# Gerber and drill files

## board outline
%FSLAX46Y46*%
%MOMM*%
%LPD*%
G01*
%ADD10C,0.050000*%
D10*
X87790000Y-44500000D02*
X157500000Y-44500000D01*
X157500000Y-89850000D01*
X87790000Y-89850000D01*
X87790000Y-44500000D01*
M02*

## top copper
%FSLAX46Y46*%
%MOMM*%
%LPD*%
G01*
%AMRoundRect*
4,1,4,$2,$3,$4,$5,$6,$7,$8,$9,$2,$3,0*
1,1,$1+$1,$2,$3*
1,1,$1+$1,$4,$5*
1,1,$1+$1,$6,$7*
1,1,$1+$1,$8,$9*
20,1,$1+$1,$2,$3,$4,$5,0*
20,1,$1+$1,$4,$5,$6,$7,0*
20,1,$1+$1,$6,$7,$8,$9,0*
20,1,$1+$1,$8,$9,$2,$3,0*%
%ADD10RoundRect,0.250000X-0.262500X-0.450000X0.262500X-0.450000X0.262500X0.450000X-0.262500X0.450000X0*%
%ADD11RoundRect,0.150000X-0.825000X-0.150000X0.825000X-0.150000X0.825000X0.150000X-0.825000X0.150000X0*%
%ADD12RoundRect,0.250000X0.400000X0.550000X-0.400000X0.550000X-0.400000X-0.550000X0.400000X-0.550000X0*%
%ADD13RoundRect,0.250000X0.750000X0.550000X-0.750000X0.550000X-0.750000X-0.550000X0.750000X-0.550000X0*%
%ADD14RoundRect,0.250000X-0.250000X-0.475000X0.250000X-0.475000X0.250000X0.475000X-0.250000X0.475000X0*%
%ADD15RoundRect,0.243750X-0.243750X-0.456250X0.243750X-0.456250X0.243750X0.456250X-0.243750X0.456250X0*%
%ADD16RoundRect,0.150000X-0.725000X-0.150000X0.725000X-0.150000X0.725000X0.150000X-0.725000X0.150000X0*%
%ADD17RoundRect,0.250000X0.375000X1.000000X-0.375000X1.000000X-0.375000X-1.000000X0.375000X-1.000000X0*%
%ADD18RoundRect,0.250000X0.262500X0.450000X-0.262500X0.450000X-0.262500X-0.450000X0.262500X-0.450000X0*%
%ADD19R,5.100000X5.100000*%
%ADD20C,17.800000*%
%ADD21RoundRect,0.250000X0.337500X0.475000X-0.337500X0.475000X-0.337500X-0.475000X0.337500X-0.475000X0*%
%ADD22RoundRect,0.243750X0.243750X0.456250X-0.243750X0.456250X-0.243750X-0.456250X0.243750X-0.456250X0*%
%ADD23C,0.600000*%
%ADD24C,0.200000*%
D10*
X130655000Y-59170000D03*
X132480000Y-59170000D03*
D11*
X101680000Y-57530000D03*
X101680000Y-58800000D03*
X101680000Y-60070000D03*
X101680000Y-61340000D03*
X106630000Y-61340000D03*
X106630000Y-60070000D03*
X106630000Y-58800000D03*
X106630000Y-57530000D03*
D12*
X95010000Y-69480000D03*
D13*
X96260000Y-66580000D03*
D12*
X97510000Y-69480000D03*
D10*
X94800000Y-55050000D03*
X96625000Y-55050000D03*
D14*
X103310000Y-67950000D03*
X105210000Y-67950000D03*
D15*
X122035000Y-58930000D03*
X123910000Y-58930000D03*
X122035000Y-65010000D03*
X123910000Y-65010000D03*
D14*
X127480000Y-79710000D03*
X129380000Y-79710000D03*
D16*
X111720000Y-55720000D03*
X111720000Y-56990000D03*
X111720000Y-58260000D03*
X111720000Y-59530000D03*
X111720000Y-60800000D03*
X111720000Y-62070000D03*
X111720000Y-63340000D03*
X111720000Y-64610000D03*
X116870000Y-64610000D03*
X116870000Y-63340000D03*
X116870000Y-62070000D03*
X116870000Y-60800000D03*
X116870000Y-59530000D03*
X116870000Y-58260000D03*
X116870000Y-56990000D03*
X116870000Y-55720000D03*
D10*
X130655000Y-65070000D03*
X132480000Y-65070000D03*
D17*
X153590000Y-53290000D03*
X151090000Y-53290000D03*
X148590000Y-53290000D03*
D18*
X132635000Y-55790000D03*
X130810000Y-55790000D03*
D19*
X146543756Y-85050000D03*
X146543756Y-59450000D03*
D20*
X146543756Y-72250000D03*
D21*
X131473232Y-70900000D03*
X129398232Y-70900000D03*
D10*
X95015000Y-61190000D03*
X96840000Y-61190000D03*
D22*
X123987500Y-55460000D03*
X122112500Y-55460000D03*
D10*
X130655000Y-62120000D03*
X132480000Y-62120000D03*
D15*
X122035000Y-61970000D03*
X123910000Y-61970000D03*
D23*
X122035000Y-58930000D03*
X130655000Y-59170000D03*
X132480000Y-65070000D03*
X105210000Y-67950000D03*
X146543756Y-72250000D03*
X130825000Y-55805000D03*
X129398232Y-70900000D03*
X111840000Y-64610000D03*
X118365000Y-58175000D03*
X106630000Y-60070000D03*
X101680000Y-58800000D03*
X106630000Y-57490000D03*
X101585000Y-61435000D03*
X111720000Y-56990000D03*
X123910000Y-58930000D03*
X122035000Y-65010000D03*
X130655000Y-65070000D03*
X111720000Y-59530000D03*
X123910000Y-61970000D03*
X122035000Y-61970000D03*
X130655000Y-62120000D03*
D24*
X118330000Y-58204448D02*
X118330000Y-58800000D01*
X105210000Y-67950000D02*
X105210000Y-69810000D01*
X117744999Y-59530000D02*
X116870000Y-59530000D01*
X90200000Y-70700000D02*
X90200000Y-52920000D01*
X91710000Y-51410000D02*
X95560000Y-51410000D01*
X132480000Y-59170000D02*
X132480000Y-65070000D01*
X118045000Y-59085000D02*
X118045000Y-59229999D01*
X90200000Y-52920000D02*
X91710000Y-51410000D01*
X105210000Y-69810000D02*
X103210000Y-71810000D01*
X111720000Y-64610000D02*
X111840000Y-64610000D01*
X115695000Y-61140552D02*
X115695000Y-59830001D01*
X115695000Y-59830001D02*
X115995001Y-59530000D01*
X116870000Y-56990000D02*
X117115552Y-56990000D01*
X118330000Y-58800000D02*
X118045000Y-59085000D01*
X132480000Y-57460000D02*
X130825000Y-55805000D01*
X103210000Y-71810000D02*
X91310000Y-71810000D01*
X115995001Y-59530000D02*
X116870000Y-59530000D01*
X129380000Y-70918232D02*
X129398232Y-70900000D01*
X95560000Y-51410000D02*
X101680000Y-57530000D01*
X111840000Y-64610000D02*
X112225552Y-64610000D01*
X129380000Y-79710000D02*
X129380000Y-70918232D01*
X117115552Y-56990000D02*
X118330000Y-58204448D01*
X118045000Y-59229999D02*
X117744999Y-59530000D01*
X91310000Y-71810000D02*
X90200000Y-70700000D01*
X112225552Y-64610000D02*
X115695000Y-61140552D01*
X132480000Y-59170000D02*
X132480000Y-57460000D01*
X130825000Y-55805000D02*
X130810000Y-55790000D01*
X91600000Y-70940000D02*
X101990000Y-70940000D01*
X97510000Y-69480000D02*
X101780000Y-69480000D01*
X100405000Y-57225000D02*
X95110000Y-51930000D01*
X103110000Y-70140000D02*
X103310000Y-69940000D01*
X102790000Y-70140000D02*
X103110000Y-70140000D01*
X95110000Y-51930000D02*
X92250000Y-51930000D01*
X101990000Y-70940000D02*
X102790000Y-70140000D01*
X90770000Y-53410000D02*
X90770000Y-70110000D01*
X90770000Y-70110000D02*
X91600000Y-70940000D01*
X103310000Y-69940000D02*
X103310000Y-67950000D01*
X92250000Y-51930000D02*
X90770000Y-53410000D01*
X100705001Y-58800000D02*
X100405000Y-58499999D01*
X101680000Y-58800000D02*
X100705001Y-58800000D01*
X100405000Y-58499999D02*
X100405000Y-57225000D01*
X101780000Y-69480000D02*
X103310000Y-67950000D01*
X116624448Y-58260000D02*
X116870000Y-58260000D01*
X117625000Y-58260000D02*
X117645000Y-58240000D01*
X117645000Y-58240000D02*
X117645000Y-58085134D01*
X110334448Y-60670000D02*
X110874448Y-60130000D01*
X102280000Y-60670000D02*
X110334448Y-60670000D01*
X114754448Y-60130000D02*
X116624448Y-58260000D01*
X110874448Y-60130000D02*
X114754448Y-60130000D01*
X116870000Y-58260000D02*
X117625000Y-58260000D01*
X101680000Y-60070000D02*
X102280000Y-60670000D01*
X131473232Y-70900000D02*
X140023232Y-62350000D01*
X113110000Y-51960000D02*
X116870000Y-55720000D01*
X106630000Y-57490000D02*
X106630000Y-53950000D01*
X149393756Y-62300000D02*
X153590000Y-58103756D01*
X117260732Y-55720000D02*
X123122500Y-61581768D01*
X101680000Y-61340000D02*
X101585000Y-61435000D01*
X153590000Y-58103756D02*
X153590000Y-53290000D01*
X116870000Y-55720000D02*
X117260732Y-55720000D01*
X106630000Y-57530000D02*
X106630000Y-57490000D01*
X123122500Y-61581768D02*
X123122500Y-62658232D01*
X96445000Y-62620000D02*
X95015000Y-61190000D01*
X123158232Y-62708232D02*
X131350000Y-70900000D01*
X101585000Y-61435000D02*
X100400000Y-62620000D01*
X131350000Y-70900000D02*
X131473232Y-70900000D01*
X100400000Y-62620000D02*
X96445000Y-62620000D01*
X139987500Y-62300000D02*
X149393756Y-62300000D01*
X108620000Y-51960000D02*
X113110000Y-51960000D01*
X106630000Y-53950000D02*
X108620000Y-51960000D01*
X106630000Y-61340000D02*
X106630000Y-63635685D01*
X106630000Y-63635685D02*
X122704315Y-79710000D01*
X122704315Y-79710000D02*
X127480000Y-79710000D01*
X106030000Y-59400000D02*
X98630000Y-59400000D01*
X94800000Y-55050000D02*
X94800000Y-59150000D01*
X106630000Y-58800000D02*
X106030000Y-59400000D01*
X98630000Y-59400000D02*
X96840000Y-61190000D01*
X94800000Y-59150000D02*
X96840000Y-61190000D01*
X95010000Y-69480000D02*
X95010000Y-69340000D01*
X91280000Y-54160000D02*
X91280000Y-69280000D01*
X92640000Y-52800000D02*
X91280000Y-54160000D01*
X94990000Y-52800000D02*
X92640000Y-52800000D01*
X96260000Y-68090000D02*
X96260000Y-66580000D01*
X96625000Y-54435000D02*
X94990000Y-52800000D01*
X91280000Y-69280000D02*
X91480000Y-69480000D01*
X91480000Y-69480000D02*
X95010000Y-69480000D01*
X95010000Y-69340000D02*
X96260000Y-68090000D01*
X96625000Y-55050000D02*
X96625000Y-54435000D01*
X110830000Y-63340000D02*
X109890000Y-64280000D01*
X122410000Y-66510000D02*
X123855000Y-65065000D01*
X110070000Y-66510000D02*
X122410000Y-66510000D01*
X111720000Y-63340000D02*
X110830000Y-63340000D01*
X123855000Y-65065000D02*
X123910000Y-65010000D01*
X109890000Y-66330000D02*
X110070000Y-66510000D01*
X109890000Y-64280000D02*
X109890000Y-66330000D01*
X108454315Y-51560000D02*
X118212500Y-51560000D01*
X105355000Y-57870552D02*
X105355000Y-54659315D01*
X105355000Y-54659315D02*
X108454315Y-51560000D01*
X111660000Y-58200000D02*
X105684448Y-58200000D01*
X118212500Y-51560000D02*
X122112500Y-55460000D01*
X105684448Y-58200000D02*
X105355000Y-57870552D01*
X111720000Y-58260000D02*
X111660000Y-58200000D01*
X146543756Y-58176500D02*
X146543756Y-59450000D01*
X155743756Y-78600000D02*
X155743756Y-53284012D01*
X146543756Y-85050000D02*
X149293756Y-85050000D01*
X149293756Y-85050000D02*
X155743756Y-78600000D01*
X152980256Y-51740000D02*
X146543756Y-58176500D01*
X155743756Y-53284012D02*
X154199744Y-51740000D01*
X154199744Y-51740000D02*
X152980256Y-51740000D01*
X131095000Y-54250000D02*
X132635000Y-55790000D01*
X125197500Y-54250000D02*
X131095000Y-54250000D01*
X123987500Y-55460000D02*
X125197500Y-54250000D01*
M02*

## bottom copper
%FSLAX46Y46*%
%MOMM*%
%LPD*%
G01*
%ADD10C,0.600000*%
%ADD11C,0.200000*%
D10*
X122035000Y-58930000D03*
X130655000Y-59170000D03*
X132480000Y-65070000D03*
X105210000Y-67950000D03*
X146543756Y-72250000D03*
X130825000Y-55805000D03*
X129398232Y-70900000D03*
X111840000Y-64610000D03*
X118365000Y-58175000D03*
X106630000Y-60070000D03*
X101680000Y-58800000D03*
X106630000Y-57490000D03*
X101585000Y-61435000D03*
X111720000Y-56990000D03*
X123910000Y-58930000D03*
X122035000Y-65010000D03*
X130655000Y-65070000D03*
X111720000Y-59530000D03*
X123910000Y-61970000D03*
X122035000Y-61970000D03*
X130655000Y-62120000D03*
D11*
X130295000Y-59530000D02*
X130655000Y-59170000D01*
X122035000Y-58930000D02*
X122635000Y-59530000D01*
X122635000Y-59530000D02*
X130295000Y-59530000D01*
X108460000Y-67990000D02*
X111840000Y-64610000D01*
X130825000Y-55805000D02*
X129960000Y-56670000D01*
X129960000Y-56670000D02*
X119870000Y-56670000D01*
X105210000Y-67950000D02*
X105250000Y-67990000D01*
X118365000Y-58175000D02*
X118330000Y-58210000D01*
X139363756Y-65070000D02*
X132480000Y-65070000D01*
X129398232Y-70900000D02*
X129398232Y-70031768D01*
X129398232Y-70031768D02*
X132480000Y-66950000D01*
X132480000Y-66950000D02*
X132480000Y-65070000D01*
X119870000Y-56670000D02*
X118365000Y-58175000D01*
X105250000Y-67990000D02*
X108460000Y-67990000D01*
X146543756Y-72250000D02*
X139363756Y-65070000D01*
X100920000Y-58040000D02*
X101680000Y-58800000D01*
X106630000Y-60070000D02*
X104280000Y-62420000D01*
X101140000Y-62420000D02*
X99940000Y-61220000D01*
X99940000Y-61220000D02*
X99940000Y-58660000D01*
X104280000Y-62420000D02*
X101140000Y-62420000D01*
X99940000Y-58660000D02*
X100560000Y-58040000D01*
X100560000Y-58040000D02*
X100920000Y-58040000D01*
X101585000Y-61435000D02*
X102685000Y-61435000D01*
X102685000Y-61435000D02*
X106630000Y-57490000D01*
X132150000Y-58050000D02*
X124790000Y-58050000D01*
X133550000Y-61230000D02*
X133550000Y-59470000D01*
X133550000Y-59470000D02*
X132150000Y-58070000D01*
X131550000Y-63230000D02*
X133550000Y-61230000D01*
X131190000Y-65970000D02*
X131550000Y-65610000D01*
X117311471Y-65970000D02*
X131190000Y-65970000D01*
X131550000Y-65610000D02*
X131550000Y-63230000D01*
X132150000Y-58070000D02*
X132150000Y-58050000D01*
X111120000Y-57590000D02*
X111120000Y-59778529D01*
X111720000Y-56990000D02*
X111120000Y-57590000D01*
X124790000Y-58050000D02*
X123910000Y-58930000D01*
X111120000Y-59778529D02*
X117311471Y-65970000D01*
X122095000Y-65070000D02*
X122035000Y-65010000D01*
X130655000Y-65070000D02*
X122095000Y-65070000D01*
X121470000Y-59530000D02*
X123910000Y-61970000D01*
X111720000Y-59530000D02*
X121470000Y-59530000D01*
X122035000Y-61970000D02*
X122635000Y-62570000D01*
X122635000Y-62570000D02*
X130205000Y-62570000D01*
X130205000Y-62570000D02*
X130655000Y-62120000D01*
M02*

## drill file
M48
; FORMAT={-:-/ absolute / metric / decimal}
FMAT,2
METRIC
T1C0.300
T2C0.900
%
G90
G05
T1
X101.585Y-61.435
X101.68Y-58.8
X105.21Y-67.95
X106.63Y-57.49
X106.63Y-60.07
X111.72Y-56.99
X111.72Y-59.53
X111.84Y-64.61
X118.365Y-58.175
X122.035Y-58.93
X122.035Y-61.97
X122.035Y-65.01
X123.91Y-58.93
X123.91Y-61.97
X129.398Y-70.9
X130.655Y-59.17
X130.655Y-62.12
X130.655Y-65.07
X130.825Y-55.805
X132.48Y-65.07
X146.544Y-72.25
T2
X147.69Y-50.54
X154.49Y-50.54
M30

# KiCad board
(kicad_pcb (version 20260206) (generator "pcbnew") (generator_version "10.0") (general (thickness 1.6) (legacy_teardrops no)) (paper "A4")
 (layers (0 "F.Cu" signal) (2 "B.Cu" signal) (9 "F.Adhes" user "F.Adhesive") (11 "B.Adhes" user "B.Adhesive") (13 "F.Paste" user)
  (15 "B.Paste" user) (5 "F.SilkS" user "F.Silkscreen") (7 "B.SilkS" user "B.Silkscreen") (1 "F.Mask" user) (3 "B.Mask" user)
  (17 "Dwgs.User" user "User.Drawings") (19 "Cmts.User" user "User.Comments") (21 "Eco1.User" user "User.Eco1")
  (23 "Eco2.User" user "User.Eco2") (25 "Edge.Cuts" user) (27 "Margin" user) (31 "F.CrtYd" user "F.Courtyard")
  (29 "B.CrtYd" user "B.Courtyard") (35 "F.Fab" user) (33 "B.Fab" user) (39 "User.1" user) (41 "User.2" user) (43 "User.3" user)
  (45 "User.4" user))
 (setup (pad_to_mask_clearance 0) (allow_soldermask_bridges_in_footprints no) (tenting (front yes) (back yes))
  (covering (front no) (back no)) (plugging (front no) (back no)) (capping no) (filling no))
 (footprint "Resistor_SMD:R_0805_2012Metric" (layer "F.Cu") (at 131.5675 59.17)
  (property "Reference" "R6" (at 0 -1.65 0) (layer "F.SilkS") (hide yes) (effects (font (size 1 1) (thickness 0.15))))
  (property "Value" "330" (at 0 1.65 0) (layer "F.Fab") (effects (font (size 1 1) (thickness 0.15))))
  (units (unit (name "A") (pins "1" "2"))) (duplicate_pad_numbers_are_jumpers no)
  (pad "1" smd roundrect (at -0.9125 0) (size 1.025 1.4) (layers "F.Cu" "F.Mask" "F.Paste") (roundrect_rratio 0.243902) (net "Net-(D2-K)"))
  (pad "2" smd roundrect (at 0.9125 0) (size 1.025 1.4) (layers "F.Cu" "F.Mask" "F.Paste") (roundrect_rratio 0.243902) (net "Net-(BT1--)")))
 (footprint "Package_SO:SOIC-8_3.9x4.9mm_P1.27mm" (layer "F.Cu") (at 104.155 59.435)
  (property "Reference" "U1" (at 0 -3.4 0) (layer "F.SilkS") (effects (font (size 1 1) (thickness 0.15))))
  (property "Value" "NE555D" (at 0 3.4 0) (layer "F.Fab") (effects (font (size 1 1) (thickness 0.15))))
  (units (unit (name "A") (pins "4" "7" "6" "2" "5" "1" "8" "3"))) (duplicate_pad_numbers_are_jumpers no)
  (pad "1" smd roundrect (at -2.475 -1.905) (size 1.95 0.6) (layers "F.Cu" "F.Mask" "F.Paste") (roundrect_rratio 0.25) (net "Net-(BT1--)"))
  (pad "2" smd roundrect (at -2.475 -0.635) (size 1.95 0.6) (layers "F.Cu" "F.Mask" "F.Paste") (roundrect_rratio 0.25)
   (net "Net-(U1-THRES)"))
  (pad "3" smd roundrect (at -2.475 0.635) (size 1.95 0.6) (layers "F.Cu" "F.Mask" "F.Paste") (roundrect_rratio 0.25) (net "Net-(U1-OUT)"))
  (pad "4" smd roundrect (at -2.475 1.905) (size 1.95 0.6) (layers "F.Cu" "F.Mask" "F.Paste") (roundrect_rratio 0.25) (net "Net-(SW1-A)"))
  (pad "5" smd roundrect (at 2.475 1.905) (size 1.95 0.6) (layers "F.Cu" "F.Mask" "F.Paste") (roundrect_rratio 0.25) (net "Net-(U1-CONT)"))
  (pad "6" smd roundrect (at 2.475 0.635) (size 1.95 0.6) (layers "F.Cu" "F.Mask" "F.Paste") (roundrect_rratio 0.25) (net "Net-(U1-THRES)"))
  (pad "7" smd roundrect (at 2.475 -0.635) (size 1.95 0.6) (layers "F.Cu" "F.Mask" "F.Paste") (roundrect_rratio 0.25) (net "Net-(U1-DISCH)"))
  (pad "8" smd roundrect (at 2.475 -1.905) (size 1.95 0.6) (layers "F.Cu" "F.Mask" "F.Paste") (roundrect_rratio 0.25) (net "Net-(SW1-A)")))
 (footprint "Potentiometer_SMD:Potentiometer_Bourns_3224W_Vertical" (layer "F.Cu") (at 96.26 68.03 180)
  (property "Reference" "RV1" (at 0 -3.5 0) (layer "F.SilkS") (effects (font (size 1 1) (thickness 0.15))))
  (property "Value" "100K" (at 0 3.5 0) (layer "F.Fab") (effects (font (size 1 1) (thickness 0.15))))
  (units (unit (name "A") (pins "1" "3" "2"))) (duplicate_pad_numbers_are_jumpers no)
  (pad "1" smd roundrect (at 1.25 -1.45 180) (size 1.3 1.6) (layers "F.Cu" "F.Mask" "F.Paste") (roundrect_rratio 0.192308)
   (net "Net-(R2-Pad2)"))
  (pad "2" smd roundrect (at 0 1.45 180) (size 2 1.6) (layers "F.Cu" "F.Mask" "F.Paste") (roundrect_rratio 0.15625) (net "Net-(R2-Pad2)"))
  (pad "3" smd roundrect (at -1.25 -1.45 180) (size 1.3 1.6) (layers "F.Cu" "F.Mask" "F.Paste") (roundrect_rratio 0.192308)
   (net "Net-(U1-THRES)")))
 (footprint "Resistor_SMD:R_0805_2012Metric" (layer "F.Cu") (at 95.7125 55.05)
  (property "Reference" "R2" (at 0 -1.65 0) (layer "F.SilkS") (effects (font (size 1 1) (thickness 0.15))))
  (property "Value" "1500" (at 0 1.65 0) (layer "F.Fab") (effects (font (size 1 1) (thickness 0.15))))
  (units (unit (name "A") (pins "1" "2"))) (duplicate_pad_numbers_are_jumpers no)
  (pad "1" smd roundrect (at -0.9125 0) (size 1.025 1.4) (layers "F.Cu" "F.Mask" "F.Paste") (roundrect_rratio 0.243902)
   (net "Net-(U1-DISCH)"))
  (pad "2" smd roundrect (at 0.9125 0) (size 1.025 1.4) (layers "F.Cu" "F.Mask" "F.Paste") (roundrect_rratio 0.243902) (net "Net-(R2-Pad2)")))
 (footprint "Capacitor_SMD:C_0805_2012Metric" (layer "F.Cu") (at 104.26 67.95)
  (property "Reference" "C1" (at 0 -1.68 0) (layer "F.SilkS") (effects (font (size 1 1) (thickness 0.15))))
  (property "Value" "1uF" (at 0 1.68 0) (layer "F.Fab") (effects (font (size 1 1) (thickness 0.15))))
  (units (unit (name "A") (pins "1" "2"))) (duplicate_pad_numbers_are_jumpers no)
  (pad "1" smd roundrect (at -0.95 0) (size 1 1.45) (layers "F.Cu" "F.Mask" "F.Paste") (roundrect_rratio 0.25) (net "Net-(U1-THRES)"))
  (pad "2" smd roundrect (at 0.95 0) (size 1 1.45) (layers "F.Cu" "F.Mask" "F.Paste") (roundrect_rratio 0.25) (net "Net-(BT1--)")))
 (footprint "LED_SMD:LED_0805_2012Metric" (layer "F.Cu") (at 122.9725 58.93)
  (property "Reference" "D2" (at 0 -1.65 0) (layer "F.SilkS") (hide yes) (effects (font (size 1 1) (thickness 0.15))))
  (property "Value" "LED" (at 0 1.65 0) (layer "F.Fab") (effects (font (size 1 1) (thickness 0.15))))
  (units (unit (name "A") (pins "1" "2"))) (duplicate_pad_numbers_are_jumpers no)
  (pad "1" smd roundrect (at -0.9375 0) (size 0.975 1.4) (layers "F.Cu" "F.Mask" "F.Paste") (roundrect_rratio 0.25) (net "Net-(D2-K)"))
  (pad "2" smd roundrect (at 0.9375 0) (size 0.975 1.4) (layers "F.Cu" "F.Mask" "F.Paste") (roundrect_rratio 0.25) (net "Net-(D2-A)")))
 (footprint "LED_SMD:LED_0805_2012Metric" (layer "F.Cu") (at 122.9725 65.01)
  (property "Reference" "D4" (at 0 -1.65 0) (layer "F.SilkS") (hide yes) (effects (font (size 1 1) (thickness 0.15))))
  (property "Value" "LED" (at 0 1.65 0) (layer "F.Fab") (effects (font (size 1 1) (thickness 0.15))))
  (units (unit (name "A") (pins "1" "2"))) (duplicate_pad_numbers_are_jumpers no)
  (pad "1" smd roundrect (at -0.9375 0) (size 0.975 1.4) (layers "F.Cu" "F.Mask" "F.Paste") (roundrect_rratio 0.25) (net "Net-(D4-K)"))
  (pad "2" smd roundrect (at 0.9375 0) (size 0.975 1.4) (layers "F.Cu" "F.Mask" "F.Paste") (roundrect_rratio 0.25) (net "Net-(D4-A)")))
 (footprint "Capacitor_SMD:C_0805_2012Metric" (layer "F.Cu") (at 128.43 79.71)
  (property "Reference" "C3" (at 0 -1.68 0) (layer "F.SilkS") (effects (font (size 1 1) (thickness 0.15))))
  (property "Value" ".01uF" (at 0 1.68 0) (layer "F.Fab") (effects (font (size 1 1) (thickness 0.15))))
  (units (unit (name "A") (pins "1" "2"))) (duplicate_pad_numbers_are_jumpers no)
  (pad "1" smd roundrect (at -0.95 0) (size 1 1.45) (layers "F.Cu" "F.Mask" "F.Paste") (roundrect_rratio 0.25) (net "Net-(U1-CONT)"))
  (pad "2" smd roundrect (at 0.95 0) (size 1 1.45) (layers "F.Cu" "F.Mask" "F.Paste") (roundrect_rratio 0.25) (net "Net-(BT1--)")))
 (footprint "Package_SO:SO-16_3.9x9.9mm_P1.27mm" (layer "F.Cu") (at 114.295 60.165)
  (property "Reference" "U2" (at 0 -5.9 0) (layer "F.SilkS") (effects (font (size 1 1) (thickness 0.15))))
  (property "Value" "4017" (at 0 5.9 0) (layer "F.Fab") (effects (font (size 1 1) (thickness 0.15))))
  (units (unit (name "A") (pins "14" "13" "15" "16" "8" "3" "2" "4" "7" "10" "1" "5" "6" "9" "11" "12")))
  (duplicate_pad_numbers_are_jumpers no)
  (pad "1" smd roundrect (at -2.575 -4.445) (size 1.75 0.6) (layers "F.Cu" "F.Mask" "F.Paste") (roundrect_rratio 0.25)
   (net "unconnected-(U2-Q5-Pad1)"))
  (pad "2" smd roundrect (at -2.575 -3.175) (size 1.75 0.6) (layers "F.Cu" "F.Mask" "F.Paste") (roundrect_rratio 0.25) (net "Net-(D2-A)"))
  (pad "3" smd roundrect (at -2.575 -1.905) (size 1.75 0.6) (layers "F.Cu" "F.Mask" "F.Paste") (roundrect_rratio 0.25) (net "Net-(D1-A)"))
  (pad "4" smd roundrect (at -2.575 -0.635) (size 1.75 0.6) (layers "F.Cu" "F.Mask" "F.Paste") (roundrect_rratio 0.25) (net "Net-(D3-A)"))
  (pad "5" smd roundrect (at -2.575 0.635) (size 1.75 0.6) (layers "F.Cu" "F.Mask" "F.Paste") (roundrect_rratio 0.25)
   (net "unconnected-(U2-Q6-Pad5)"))
  (pad "6" smd roundrect (at -2.575 1.905) (size 1.75 0.6) (layers "F.Cu" "F.Mask" "F.Paste") (roundrect_rratio 0.25)
   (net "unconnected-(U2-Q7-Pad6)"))
  (pad "7" smd roundrect (at -2.575 3.175) (size 1.75 0.6) (layers "F.Cu" "F.Mask" "F.Paste") (roundrect_rratio 0.25) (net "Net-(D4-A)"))
  (pad "8" smd roundrect (at -2.575 4.445) (size 1.75 0.6) (layers "F.Cu" "F.Mask" "F.Paste") (roundrect_rratio 0.25) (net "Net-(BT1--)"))
  (pad "9" smd roundrect (at 2.575 4.445) (size 1.75 0.6) (layers "F.Cu" "F.Mask" "F.Paste") (roundrect_rratio 0.25)
   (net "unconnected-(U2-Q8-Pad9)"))
  (pad "10" smd roundrect (at 2.575 3.175) (size 1.75 0.6) (layers "F.Cu" "F.Mask" "F.Paste") (roundrect_rratio 0.25)
   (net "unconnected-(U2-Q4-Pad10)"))
  (pad "11" smd roundrect (at 2.575 1.905) (size 1.75 0.6) (layers "F.Cu" "F.Mask" "F.Paste") (roundrect_rratio 0.25)
   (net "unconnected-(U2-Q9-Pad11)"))
  (pad "12" smd roundrect (at 2.575 0.635) (size 1.75 0.6) (layers "F.Cu" "F.Mask" "F.Paste") (roundrect_rratio 0.25)
   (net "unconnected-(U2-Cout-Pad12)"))
  (pad "13" smd roundrect (at 2.575 -0.635) (size 1.75 0.6) (layers "F.Cu" "F.Mask" "F.Paste") (roundrect_rratio 0.25) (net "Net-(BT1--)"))
  (pad "14" smd roundrect (at 2.575 -1.905) (size 1.75 0.6) (layers "F.Cu" "F.Mask" "F.Paste") (roundrect_rratio 0.25) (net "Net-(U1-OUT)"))
  (pad "15" smd roundrect (at 2.575 -3.175) (size 1.75 0.6) (layers "F.Cu" "F.Mask" "F.Paste") (roundrect_rratio 0.25) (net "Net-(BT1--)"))
  (pad "16" smd roundrect (at 2.575 -4.445) (size 1.75 0.6) (layers "F.Cu" "F.Mask" "F.Paste") (roundrect_rratio 0.25) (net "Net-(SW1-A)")))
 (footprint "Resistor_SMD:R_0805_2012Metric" (layer "F.Cu") (at 131.5675 65.07)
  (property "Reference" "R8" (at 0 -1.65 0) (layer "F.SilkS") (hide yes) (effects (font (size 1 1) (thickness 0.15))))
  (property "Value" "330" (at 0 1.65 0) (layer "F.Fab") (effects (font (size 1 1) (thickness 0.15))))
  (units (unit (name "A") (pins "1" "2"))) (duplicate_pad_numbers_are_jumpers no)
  (pad "1" smd roundrect (at -0.9125 0) (size 1.025 1.4) (layers "F.Cu" "F.Mask" "F.Paste") (roundrect_rratio 0.243902) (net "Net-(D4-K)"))
  (pad "2" smd roundrect (at 0.9125 0) (size 1.025 1.4) (layers "F.Cu" "F.Mask" "F.Paste") (roundrect_rratio 0.243902) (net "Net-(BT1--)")))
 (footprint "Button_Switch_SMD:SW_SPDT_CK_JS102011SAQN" (layer "F.Cu") (at 151.09 50.54 180)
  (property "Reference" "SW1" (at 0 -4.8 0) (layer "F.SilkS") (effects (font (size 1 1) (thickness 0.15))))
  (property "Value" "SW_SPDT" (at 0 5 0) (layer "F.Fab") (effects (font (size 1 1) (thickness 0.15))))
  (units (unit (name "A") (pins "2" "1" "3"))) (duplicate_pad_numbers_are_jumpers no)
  (pad "" np_thru_hole circle (at -3.4 0 180) (size 0.9 0.9) (drill 0.9) (layers "*.Cu" "*.Mask"))
  (pad "" np_thru_hole circle (at 3.4 0 180) (size 0.9 0.9) (drill 0.9) (layers "*.Cu" "*.Mask"))
  (pad "1" smd roundrect (at -2.5 -2.75 180) (size 1.25 2.5) (layers "F.Cu" "F.Mask" "F.Paste") (roundrect_rratio 0.2) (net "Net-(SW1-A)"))
  (pad "2" smd roundrect (at 0 -2.75 180) (size 1.25 2.5) (layers "F.Cu" "F.Mask" "F.Paste") (roundrect_rratio 0.2) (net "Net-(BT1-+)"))
  (pad "3" smd roundrect (at 2.5 -2.75 180) (size 1.25 2.5) (layers "F.Cu" "F.Mask" "F.Paste") (roundrect_rratio 0.2)
   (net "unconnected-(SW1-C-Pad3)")))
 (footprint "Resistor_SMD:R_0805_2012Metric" (layer "F.Cu") (at 131.7225 55.79 180)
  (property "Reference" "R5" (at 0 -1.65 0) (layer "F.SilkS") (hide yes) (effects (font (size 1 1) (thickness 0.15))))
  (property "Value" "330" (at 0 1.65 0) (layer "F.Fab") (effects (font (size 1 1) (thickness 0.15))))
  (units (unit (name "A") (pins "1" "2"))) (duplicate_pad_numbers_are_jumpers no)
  (pad "1" smd roundrect (at -0.9125 0 180) (size 1.025 1.4) (layers "F.Cu" "F.Mask" "F.Paste") (roundrect_rratio 0.243902)
   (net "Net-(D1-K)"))
  (pad "2" smd roundrect (at 0.9125 0 180) (size 1.025 1.4) (layers "F.Cu" "F.Mask" "F.Paste") (roundrect_rratio 0.243902)
   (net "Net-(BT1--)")))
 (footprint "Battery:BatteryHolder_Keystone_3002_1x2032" (layer "F.Cu") (at 146.543756 72.25 90)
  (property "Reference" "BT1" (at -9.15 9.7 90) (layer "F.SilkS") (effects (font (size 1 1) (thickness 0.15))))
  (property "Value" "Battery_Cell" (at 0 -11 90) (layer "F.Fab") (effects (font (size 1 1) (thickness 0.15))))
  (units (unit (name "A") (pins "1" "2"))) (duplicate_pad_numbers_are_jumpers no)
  (pad "1" smd rect (at -12.8 0 90) (size 5.1 5.1) (layers "F.Cu" "F.Mask" "F.Paste") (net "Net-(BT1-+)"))
  (pad "1" smd rect (at 12.8 0 90) (size 5.1 5.1) (layers "F.Cu" "F.Mask" "F.Paste") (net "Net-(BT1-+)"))
  (pad "2" smd circle (at 0 0 90) (size 17.8 17.8) (layers "F.Cu" "F.Mask") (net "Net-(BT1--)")))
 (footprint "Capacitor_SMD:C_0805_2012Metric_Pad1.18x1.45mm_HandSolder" (layer "F.Cu") (at 130.435732 70.9 180)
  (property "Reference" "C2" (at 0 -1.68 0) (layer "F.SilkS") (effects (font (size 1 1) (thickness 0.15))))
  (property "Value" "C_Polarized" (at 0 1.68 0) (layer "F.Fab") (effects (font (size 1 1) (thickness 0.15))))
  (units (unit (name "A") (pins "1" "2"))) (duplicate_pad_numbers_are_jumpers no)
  (pad "1" smd roundrect (at -1.0375 0 180) (size 1.175 1.45) (layers "F.Cu" "F.Mask" "F.Paste") (roundrect_rratio 0.212766)
   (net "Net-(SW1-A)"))
  (pad "2" smd roundrect (at 1.0375 0 180) (size 1.175 1.45) (layers "F.Cu" "F.Mask" "F.Paste") (roundrect_rratio 0.212766)
   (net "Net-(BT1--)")))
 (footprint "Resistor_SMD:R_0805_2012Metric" (layer "F.Cu") (at 95.9275 61.19)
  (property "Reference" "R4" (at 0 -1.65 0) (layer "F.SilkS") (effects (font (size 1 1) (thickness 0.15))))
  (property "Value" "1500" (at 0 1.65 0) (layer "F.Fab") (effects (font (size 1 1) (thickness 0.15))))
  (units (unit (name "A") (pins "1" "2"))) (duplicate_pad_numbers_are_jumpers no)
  (pad "1" smd roundrect (at -0.9125 0) (size 1.025 1.4) (layers "F.Cu" "F.Mask" "F.Paste") (roundrect_rratio 0.243902) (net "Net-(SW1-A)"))
  (pad "2" smd roundrect (at 0.9125 0) (size 1.025 1.4) (layers "F.Cu" "F.Mask" "F.Paste") (roundrect_rratio 0.243902)
   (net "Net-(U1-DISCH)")))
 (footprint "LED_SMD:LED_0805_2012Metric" (layer "F.Cu") (at 123.05 55.46 180)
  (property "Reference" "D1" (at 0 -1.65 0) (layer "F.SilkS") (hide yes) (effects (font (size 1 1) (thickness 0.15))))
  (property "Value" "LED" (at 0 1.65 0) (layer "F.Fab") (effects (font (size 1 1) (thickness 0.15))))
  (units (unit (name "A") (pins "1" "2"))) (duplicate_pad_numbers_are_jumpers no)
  (pad "1" smd roundrect (at -0.9375 0 180) (size 0.975 1.4) (layers "F.Cu" "F.Mask" "F.Paste") (roundrect_rratio 0.25) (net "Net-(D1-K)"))
  (pad "2" smd roundrect (at 0.9375 0 180) (size 0.975 1.4) (layers "F.Cu" "F.Mask" "F.Paste") (roundrect_rratio 0.25) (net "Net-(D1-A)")))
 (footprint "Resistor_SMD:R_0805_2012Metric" (layer "F.Cu") (at 131.5675 62.12)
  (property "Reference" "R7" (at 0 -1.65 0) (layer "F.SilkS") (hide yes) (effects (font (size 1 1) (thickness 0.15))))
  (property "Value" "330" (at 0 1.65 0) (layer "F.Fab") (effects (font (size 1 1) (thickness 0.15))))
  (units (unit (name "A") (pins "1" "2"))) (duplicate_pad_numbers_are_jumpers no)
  (pad "1" smd roundrect (at -0.9125 0) (size 1.025 1.4) (layers "F.Cu" "F.Mask" "F.Paste") (roundrect_rratio 0.243902) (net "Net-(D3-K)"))
  (pad "2" smd roundrect (at 0.9125 0) (size 1.025 1.4) (layers "F.Cu" "F.Mask" "F.Paste") (roundrect_rratio 0.243902) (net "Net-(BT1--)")))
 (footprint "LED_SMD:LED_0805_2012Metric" (layer "F.Cu") (at 122.9725 61.97)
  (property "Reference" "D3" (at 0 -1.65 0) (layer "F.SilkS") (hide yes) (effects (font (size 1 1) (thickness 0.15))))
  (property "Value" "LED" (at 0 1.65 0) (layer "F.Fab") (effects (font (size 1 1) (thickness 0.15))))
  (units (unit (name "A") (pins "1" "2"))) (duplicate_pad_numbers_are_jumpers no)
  (pad "1" smd roundrect (at -0.9375 0) (size 0.975 1.4) (layers "F.Cu" "F.Mask" "F.Paste") (roundrect_rratio 0.25) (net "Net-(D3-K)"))
  (pad "2" smd roundrect (at 0.9375 0) (size 0.975 1.4) (layers "F.Cu" "F.Mask" "F.Paste") (roundrect_rratio 0.25) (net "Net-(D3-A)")))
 (gr_rect (start 87.79 44.5) (end 157.5 89.85) (stroke (width 0.05) (type default)) (fill no) (layer "Edge.Cuts"))
 (via (at 122.035 58.93) (size 0.6) (drill 0.3) (layers "F.Cu" "B.Cu") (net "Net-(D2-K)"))
 (via (at 130.655 59.17) (size 0.6) (drill 0.3) (layers "F.Cu" "B.Cu") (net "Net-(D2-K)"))
 (segment (start 130.295 59.53) (end 130.655 59.17) (width 0.2) (layer "B.Cu") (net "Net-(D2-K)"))
 (segment (start 122.035 58.93) (end 122.635 59.53) (width 0.2) (layer "B.Cu") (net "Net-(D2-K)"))
 (segment (start 122.635 59.53) (end 130.295 59.53) (width 0.2) (layer "B.Cu") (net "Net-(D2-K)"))
 (segment (start 118.33 58.204448) (end 118.33 58.8) (width 0.2) (layer "F.Cu") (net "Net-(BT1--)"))
 (segment (start 105.21 67.95) (end 105.21 69.81) (width 0.2) (layer "F.Cu") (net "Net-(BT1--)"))
 (segment (start 117.744999 59.53) (end 116.87 59.53) (width 0.2) (layer "F.Cu") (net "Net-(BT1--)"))
 (segment (start 90.2 70.7) (end 90.2 52.92) (width 0.2) (layer "F.Cu") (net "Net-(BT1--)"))
 (segment (start 91.71 51.41) (end 95.56 51.41) (width 0.2) (layer "F.Cu") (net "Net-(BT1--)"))
 (segment (start 132.48 59.17) (end 132.48 65.07) (width 0.2) (layer "F.Cu") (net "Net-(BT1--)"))
 (segment (start 118.045 59.085) (end 118.045 59.229999) (width 0.2) (layer "F.Cu") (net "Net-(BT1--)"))
 (segment (start 90.2 52.92) (end 91.71 51.41) (width 0.2) (layer "F.Cu") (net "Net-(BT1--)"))
 (segment (start 105.21 69.81) (end 103.21 71.81) (width 0.2) (layer "F.Cu") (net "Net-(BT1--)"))
 (segment (start 111.72 64.61) (end 111.84 64.61) (width 0.2) (layer "F.Cu") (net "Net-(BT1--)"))
 (segment (start 115.695 61.140552) (end 115.695 59.830001) (width 0.2) (layer "F.Cu") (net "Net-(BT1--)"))
 (segment (start 115.695 59.830001) (end 115.995001 59.53) (width 0.2) (layer "F.Cu") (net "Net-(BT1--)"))
 (segment (start 116.87 56.99) (end 117.115552 56.99) (width 0.2) (layer "F.Cu") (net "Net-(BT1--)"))
 (segment (start 118.33 58.8) (end 118.045 59.085) (width 0.2) (layer "F.Cu") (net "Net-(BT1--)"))
 (segment (start 132.48 57.46) (end 130.825 55.805) (width 0.2) (layer "F.Cu") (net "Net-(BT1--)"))
 (segment (start 103.21 71.81) (end 91.31 71.81) (width 0.2) (layer "F.Cu") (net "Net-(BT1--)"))
 (segment (start 115.995001 59.53) (end 116.87 59.53) (width 0.2) (layer "F.Cu") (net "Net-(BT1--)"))
 (segment (start 129.38 70.918232) (end 129.398232 70.9) (width 0.2) (layer "F.Cu") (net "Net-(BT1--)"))
 (segment (start 95.56 51.41) (end 101.68 57.53) (width 0.2) (layer "F.Cu") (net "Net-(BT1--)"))
 (segment (start 111.84 64.61) (end 112.225552 64.61) (width 0.2) (layer "F.Cu") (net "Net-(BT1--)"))
 (segment (start 129.38 79.71) (end 129.38 70.918232) (width 0.2) (layer "F.Cu") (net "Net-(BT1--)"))
 (segment (start 117.115552 56.99) (end 118.33 58.204448) (width 0.2) (layer "F.Cu") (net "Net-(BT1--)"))
 (segment (start 118.045 59.229999) (end 117.744999 59.53) (width 0.2) (layer "F.Cu") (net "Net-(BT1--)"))
 (segment (start 91.31 71.81) (end 90.2 70.7) (width 0.2) (layer "F.Cu") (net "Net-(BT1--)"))
 (segment (start 112.225552 64.61) (end 115.695 61.140552) (width 0.2) (layer "F.Cu") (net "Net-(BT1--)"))
 (segment (start 132.48 59.17) (end 132.48 57.46) (width 0.2) (layer "F.Cu") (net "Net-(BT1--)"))
 (segment (start 130.825 55.805) (end 130.81 55.79) (width 0.2) (layer "F.Cu") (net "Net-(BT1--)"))
 (via (at 132.48 65.07) (size 0.6) (drill 0.3) (layers "F.Cu" "B.Cu") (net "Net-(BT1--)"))
 (via (at 105.21 67.95) (size 0.6) (drill 0.3) (layers "F.Cu" "B.Cu") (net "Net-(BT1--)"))
 (via (at 146.543756 72.25) (size 0.6) (drill 0.3) (layers "F.Cu" "B.Cu") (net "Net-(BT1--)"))
 (via (at 130.825 55.805) (size 0.6) (drill 0.3) (layers "F.Cu" "B.Cu") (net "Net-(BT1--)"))
 (via (at 129.398232 70.9) (size 0.6) (drill 0.3) (layers "F.Cu" "B.Cu") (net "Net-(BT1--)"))
 (via (at 111.84 64.61) (size 0.6) (drill 0.3) (layers "F.Cu" "B.Cu") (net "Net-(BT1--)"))
 (via (at 118.365 58.175) (size 0.6) (drill 0.3) (layers "F.Cu" "B.Cu") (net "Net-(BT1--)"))
 (segment (start 108.46 67.99) (end 111.84 64.61) (width 0.2) (layer "B.Cu") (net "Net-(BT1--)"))
 (segment (start 130.825 55.805) (end 129.96 56.67) (width 0.2) (layer "B.Cu") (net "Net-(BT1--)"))
 (segment (start 129.96 56.67) (end 119.87 56.67) (width 0.2) (layer "B.Cu") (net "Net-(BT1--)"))
 (segment (start 105.21 67.95) (end 105.25 67.99) (width 0.2) (layer "B.Cu") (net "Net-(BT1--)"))
 (segment (start 118.365 58.175) (end 118.33 58.21) (width 0.2) (layer "B.Cu") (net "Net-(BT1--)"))
 (segment (start 139.363756 65.07) (end 132.48 65.07) (width 0.2) (layer "B.Cu") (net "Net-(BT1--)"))
 (segment (start 129.398232 70.9) (end 129.398232 70.031768) (width 0.2) (layer "B.Cu") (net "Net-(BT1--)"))
 (segment (start 129.398232 70.031768) (end 132.48 66.95) (width 0.2) (layer "B.Cu") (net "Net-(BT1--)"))
 (segment (start 132.48 66.95) (end 132.48 65.07) (width 0.2) (layer "B.Cu") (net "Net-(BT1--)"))
 (segment (start 119.87 56.67) (end 118.365 58.175) (width 0.2) (layer "B.Cu") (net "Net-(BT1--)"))
 (segment (start 105.25 67.99) (end 108.46 67.99) (width 0.2) (layer "B.Cu") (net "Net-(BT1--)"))
 (segment (start 146.543756 72.25) (end 139.363756 65.07) (width 0.2) (layer "B.Cu") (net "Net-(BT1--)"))
 (segment (start 91.6 70.94) (end 101.99 70.94) (width 0.2) (layer "F.Cu") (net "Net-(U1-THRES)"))
 (segment (start 97.51 69.48) (end 101.78 69.48) (width 0.2) (layer "F.Cu") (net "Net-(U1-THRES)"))
 (segment (start 100.405 57.225) (end 95.11 51.93) (width 0.2) (layer "F.Cu") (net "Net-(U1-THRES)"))
 (segment (start 103.11 70.14) (end 103.31 69.94) (width 0.2) (layer "F.Cu") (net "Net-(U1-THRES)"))
 (segment (start 102.79 70.14) (end 103.11 70.14) (width 0.2) (layer "F.Cu") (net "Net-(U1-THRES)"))
 (segment (start 95.11 51.93) (end 92.25 51.93) (width 0.2) (layer "F.Cu") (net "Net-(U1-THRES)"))
 (segment (start 101.99 70.94) (end 102.79 70.14) (width 0.2) (layer "F.Cu") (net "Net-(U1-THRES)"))
 (segment (start 90.77 53.41) (end 90.77 70.11) (width 0.2) (layer "F.Cu") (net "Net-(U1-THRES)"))
 (segment (start 90.77 70.11) (end 91.6 70.94) (width 0.2) (layer "F.Cu") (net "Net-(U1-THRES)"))
 (segment (start 103.31 69.94) (end 103.31 67.95) (width 0.2) (layer "F.Cu") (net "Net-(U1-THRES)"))
 (segment (start 92.25 51.93) (end 90.77 53.41) (width 0.2) (layer "F.Cu") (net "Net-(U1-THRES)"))
 (segment (start 100.705001 58.8) (end 100.405 58.499999) (width 0.2) (layer "F.Cu") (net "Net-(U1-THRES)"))
 (segment (start 101.68 58.8) (end 100.705001 58.8) (width 0.2) (layer "F.Cu") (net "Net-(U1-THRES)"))
 (segment (start 100.405 58.499999) (end 100.405 57.225) (width 0.2) (layer "F.Cu") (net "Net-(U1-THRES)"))
 (segment (start 101.78 69.48) (end 103.31 67.95) (width 0.2) (layer "F.Cu") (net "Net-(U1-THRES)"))
 (via (at 106.63 60.07) (size 0.6) (drill 0.3) (layers "F.Cu" "B.Cu") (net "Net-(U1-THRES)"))
 (via (at 101.68 58.8) (size 0.6) (drill 0.3) (layers "F.Cu" "B.Cu") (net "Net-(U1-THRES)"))
 (segment (start 100.92 58.04) (end 101.68 58.8) (width 0.2) (layer "B.Cu") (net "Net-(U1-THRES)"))
 (segment (start 106.63 60.07) (end 104.28 62.42) (width 0.2) (layer "B.Cu") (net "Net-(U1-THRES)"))
 (segment (start 101.14 62.42) (end 99.94 61.22) (width 0.2) (layer "B.Cu") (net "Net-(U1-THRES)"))
 (segment (start 99.94 61.22) (end 99.94 58.66) (width 0.2) (layer "B.Cu") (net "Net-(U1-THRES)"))
 (segment (start 104.28 62.42) (end 101.14 62.42) (width 0.2) (layer "B.Cu") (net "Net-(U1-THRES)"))
 (segment (start 99.94 58.66) (end 100.56 58.04) (width 0.2) (layer "B.Cu") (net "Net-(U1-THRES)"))
 (segment (start 100.56 58.04) (end 100.92 58.04) (width 0.2) (layer "B.Cu") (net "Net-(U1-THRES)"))
 (segment (start 116.624448 58.26) (end 116.87 58.26) (width 0.2) (layer "F.Cu") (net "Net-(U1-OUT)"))
 (segment (start 117.625 58.26) (end 117.645 58.24) (width 0.2) (layer "F.Cu") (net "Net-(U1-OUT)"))
 (segment (start 117.645 58.24) (end 117.645 58.085134) (width 0.2) (layer "F.Cu") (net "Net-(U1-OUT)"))
 (segment (start 110.334448 60.67) (end 110.874448 60.13) (width 0.2) (layer "F.Cu") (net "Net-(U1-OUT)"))
 (segment (start 102.28 60.67) (end 110.334448 60.67) (width 0.2) (layer "F.Cu") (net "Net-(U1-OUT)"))
 (segment (start 114.754448 60.13) (end 116.624448 58.26) (width 0.2) (layer "F.Cu") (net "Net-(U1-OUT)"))
 (segment (start 110.874448 60.13) (end 114.754448 60.13) (width 0.2) (layer "F.Cu") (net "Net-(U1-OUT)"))
 (segment (start 116.87 58.26) (end 117.625 58.26) (width 0.2) (layer "F.Cu") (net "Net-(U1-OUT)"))
 (segment (start 101.68 60.07) (end 102.28 60.67) (width 0.2) (layer "F.Cu") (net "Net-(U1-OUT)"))
 (segment (start 131.473232 70.9) (end 140.023232 62.35) (width 0.2) (layer "F.Cu") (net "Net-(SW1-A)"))
 (segment (start 113.11 51.96) (end 116.87 55.72) (width 0.2) (layer "F.Cu") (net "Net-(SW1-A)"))
 (segment (start 106.63 57.49) (end 106.63 53.95) (width 0.2) (layer "F.Cu") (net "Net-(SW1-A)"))
 (segment (start 149.393756 62.3) (end 153.59 58.103756) (width 0.2) (layer "F.Cu") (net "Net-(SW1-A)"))
 (segment (start 117.260732 55.72) (end 123.1225 61.581768) (width 0.2) (layer "F.Cu") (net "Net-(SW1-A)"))
 (segment (start 101.68 61.34) (end 101.585 61.435) (width 0.2) (layer "F.Cu") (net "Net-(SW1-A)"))
 (segment (start 153.59 58.103756) (end 153.59 53.29) (width 0.2) (layer "F.Cu") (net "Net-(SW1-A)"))
 (segment (start 116.87 55.72) (end 117.260732 55.72) (width 0.2) (layer "F.Cu") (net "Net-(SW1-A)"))
 (segment (start 106.63 57.53) (end 106.63 57.49) (width 0.2) (layer "F.Cu") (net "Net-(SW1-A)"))
 (segment (start 123.1225 61.581768) (end 123.1225 62.658232) (width 0.2) (layer "F.Cu") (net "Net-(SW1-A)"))
 (segment (start 96.445 62.62) (end 95.015 61.19) (width 0.2) (layer "F.Cu") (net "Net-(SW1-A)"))
 (segment (start 123.158232 62.708232) (end 131.35 70.9) (width 0.2) (layer "F.Cu") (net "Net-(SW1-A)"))
 (segment (start 101.585 61.435) (end 100.4 62.62) (width 0.2) (layer "F.Cu") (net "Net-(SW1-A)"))
 (segment (start 131.35 70.9) (end 131.473232 70.9) (width 0.2) (layer "F.Cu") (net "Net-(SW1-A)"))
 (segment (start 100.4 62.62) (end 96.445 62.62) (width 0.2) (layer "F.Cu") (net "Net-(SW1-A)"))
 (segment (start 139.9875 62.3) (end 149.393756 62.3) (width 0.2) (layer "F.Cu") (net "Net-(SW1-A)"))
 (segment (start 108.62 51.96) (end 113.11 51.96) (width 0.2) (layer "F.Cu") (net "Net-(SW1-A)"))
 (segment (start 106.63 53.95) (end 108.62 51.96) (width 0.2) (layer "F.Cu") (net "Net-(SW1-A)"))
 (via (at 106.63 57.49) (size 0.6) (drill 0.3) (layers "F.Cu" "B.Cu") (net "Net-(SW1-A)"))
 (via (at 101.585 61.435) (size 0.6) (drill 0.3) (layers "F.Cu" "B.Cu") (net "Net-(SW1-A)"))
 (segment (start 101.585 61.435) (end 102.685 61.435) (width 0.2) (layer "B.Cu") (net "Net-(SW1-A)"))
 (segment (start 102.685 61.435) (end 106.63 57.49) (width 0.2) (layer "B.Cu") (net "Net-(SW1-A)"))
 (segment (start 106.63 61.34) (end 106.63 63.635685) (width 0.2) (layer "F.Cu") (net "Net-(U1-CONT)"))
 (segment (start 106.63 63.635685) (end 122.704315 79.71) (width 0.2) (layer "F.Cu") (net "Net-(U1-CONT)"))
 (segment (start 122.704315 79.71) (end 127.48 79.71) (width 0.2) (layer "F.Cu") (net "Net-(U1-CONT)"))
 (segment (start 106.03 59.4) (end 98.63 59.4) (width 0.2) (layer "F.Cu") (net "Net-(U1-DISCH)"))
 (segment (start 94.8 55.05) (end 94.8 59.15) (width 0.2) (layer "F.Cu") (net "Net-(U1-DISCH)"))
 (segment (start 106.63 58.8) (end 106.03 59.4) (width 0.2) (layer "F.Cu") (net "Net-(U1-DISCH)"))
 (segment (start 98.63 59.4) (end 96.84 61.19) (width 0.2) (layer "F.Cu") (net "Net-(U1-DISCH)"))
 (segment (start 94.8 59.15) (end 96.84 61.19) (width 0.2) (layer "F.Cu") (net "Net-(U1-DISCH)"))
 (segment (start 95.01 69.48) (end 95.01 69.34) (width 0.2) (layer "F.Cu") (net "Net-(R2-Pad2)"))
 (segment (start 91.28 54.16) (end 91.28 69.28) (width 0.2) (layer "F.Cu") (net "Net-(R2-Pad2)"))
 (segment (start 92.64 52.8) (end 91.28 54.16) (width 0.2) (layer "F.Cu") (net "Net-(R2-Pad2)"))
 (segment (start 94.99 52.8) (end 92.64 52.8) (width 0.2) (layer "F.Cu") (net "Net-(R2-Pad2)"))
 (segment (start 96.26 68.09) (end 96.26 66.58) (width 0.2) (layer "F.Cu") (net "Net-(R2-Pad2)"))
 (segment (start 96.625 54.435) (end 94.99 52.8) (width 0.2) (layer "F.Cu") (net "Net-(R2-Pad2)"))
 (segment (start 91.28 69.28) (end 91.48 69.48) (width 0.2) (layer "F.Cu") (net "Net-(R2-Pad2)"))
 (segment (start 91.48 69.48) (end 95.01 69.48) (width 0.2) (layer "F.Cu") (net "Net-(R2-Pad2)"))
 (segment (start 95.01 69.34) (end 96.26 68.09) (width 0.2) (layer "F.Cu") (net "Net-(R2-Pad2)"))
 (segment (start 96.625 55.05) (end 96.625 54.435) (width 0.2) (layer "F.Cu") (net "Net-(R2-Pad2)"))
 (via (at 111.72 56.99) (size 0.6) (drill 0.3) (layers "F.Cu" "B.Cu") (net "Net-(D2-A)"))
 (via (at 123.91 58.93) (size 0.6) (drill 0.3) (layers "F.Cu" "B.Cu") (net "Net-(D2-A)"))
 (segment (start 132.15 58.05) (end 124.79 58.05) (width 0.2) (layer "B.Cu") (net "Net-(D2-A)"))
 (segment (start 133.55 61.23) (end 133.55 59.47) (width 0.2) (layer "B.Cu") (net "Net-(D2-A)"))
 (segment (start 133.55 59.47) (end 132.15 58.07) (width 0.2) (layer "B.Cu") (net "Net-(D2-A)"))
 (segment (start 131.55 63.23) (end 133.55 61.23) (width 0.2) (layer "B.Cu") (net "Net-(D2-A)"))
 (segment (start 131.19 65.97) (end 131.55 65.61) (width 0.2) (layer "B.Cu") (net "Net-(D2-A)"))
 (segment (start 117.311471 65.97) (end 131.19 65.97) (width 0.2) (layer "B.Cu") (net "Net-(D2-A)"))
 (segment (start 131.55 65.61) (end 131.55 63.23) (width 0.2) (layer "B.Cu") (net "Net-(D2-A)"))
 (segment (start 132.15 58.07) (end 132.15 58.05) (width 0.2) (layer "B.Cu") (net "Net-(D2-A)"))
 (segment (start 111.12 57.59) (end 111.12 59.778529) (width 0.2) (layer "B.Cu") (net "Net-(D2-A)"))
 (segment (start 111.72 56.99) (end 111.12 57.59) (width 0.2) (layer "B.Cu") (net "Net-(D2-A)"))
 (segment (start 124.79 58.05) (end 123.91 58.93) (width 0.2) (layer "B.Cu") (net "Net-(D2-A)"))
 (segment (start 111.12 59.778529) (end 117.311471 65.97) (width 0.2) (layer "B.Cu") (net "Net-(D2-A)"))
 (via (at 122.035 65.01) (size 0.6) (drill 0.3) (layers "F.Cu" "B.Cu") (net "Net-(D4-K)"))
 (via (at 130.655 65.07) (size 0.6) (drill 0.3) (layers "F.Cu" "B.Cu") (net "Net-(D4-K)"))
 (segment (start 122.095 65.07) (end 122.035 65.01) (width 0.2) (layer "B.Cu") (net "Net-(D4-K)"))
 (segment (start 130.655 65.07) (end 122.095 65.07) (width 0.2) (layer "B.Cu") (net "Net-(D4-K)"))
 (segment (start 110.83 63.34) (end 109.89 64.28) (width 0.2) (layer "F.Cu") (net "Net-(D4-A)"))
 (segment (start 122.41 66.51) (end 123.855 65.065) (width 0.2) (layer "F.Cu") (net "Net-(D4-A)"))
 (segment (start 110.07 66.51) (end 122.41 66.51) (width 0.2) (layer "F.Cu") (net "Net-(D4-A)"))
 (segment (start 111.72 63.34) (end 110.83 63.34) (width 0.2) (layer "F.Cu") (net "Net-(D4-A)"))
 (segment (start 123.855 65.065) (end 123.91 65.01) (width 0.2) (layer "F.Cu") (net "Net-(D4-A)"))
 (segment (start 109.89 66.33) (end 110.07 66.51) (width 0.2) (layer "F.Cu") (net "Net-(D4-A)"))
 (segment (start 109.89 64.28) (end 109.89 66.33) (width 0.2) (layer "F.Cu") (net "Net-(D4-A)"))
 (segment (start 108.454315 51.56) (end 118.2125 51.56) (width 0.2) (layer "F.Cu") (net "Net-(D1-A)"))
 (segment (start 105.355 57.870552) (end 105.355 54.659315) (width 0.2) (layer "F.Cu") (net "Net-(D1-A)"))
 (segment (start 105.355 54.659315) (end 108.454315 51.56) (width 0.2) (layer "F.Cu") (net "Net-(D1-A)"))
 (segment (start 111.66 58.2) (end 105.684448 58.2) (width 0.2) (layer "F.Cu") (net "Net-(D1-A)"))
 (segment (start 118.2125 51.56) (end 122.1125 55.46) (width 0.2) (layer "F.Cu") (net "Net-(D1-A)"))
 (segment (start 105.684448 58.2) (end 105.355 57.870552) (width 0.2) (layer "F.Cu") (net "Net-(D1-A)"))
 (segment (start 111.72 58.26) (end 111.66 58.2) (width 0.2) (layer "F.Cu") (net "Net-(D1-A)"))
 (via (at 111.72 59.53) (size 0.6) (drill 0.3) (layers "F.Cu" "B.Cu") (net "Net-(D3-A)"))
 (via (at 123.91 61.97) (size 0.6) (drill 0.3) (layers "F.Cu" "B.Cu") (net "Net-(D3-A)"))
 (segment (start 121.47 59.53) (end 123.91 61.97) (width 0.2) (layer "B.Cu") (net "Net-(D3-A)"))
 (segment (start 111.72 59.53) (end 121.47 59.53) (width 0.2) (layer "B.Cu") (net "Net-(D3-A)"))
 (segment (start 146.543756 58.1765) (end 146.543756 59.45) (width 0.2) (layer "F.Cu") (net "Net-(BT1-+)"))
 (segment (start 155.743756 78.6) (end 155.743756 53.284012) (width 0.2) (layer "F.Cu") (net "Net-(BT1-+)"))
 (segment (start 146.543756 85.05) (end 149.293756 85.05) (width 0.2) (layer "F.Cu") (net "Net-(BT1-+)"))
 (segment (start 149.293756 85.05) (end 155.743756 78.6) (width 0.2) (layer "F.Cu") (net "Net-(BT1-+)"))
 (segment (start 152.980256 51.74) (end 146.543756 58.1765) (width 0.2) (layer "F.Cu") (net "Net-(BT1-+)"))
 (segment (start 155.743756 53.284012) (end 154.199744 51.74) (width 0.2) (layer "F.Cu") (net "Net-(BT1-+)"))
 (segment (start 154.199744 51.74) (end 152.980256 51.74) (width 0.2) (layer "F.Cu") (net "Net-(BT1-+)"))
 (segment (start 131.095 54.25) (end 132.635 55.79) (width 0.2) (layer "F.Cu") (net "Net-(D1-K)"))
 (segment (start 125.1975 54.25) (end 131.095 54.25) (width 0.2) (layer "F.Cu") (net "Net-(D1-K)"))
 (segment (start 123.9875 55.46) (end 125.1975 54.25) (width 0.2) (layer "F.Cu") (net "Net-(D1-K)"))
 (via (at 122.035 61.97) (size 0.6) (drill 0.3) (layers "F.Cu" "B.Cu") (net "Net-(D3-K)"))
 (via (at 130.655 62.12) (size 0.6) (drill 0.3) (layers "F.Cu" "B.Cu") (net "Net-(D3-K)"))
 (segment (start 122.035 61.97) (end 122.635 62.57) (width 0.2) (layer "B.Cu") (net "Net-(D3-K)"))
 (segment (start 122.635 62.57) (end 130.205 62.57) (width 0.2) (layer "B.Cu") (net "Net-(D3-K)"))
 (segment (start 130.205 62.57) (end 130.655 62.12) (width 0.2) (layer "B.Cu") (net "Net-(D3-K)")))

